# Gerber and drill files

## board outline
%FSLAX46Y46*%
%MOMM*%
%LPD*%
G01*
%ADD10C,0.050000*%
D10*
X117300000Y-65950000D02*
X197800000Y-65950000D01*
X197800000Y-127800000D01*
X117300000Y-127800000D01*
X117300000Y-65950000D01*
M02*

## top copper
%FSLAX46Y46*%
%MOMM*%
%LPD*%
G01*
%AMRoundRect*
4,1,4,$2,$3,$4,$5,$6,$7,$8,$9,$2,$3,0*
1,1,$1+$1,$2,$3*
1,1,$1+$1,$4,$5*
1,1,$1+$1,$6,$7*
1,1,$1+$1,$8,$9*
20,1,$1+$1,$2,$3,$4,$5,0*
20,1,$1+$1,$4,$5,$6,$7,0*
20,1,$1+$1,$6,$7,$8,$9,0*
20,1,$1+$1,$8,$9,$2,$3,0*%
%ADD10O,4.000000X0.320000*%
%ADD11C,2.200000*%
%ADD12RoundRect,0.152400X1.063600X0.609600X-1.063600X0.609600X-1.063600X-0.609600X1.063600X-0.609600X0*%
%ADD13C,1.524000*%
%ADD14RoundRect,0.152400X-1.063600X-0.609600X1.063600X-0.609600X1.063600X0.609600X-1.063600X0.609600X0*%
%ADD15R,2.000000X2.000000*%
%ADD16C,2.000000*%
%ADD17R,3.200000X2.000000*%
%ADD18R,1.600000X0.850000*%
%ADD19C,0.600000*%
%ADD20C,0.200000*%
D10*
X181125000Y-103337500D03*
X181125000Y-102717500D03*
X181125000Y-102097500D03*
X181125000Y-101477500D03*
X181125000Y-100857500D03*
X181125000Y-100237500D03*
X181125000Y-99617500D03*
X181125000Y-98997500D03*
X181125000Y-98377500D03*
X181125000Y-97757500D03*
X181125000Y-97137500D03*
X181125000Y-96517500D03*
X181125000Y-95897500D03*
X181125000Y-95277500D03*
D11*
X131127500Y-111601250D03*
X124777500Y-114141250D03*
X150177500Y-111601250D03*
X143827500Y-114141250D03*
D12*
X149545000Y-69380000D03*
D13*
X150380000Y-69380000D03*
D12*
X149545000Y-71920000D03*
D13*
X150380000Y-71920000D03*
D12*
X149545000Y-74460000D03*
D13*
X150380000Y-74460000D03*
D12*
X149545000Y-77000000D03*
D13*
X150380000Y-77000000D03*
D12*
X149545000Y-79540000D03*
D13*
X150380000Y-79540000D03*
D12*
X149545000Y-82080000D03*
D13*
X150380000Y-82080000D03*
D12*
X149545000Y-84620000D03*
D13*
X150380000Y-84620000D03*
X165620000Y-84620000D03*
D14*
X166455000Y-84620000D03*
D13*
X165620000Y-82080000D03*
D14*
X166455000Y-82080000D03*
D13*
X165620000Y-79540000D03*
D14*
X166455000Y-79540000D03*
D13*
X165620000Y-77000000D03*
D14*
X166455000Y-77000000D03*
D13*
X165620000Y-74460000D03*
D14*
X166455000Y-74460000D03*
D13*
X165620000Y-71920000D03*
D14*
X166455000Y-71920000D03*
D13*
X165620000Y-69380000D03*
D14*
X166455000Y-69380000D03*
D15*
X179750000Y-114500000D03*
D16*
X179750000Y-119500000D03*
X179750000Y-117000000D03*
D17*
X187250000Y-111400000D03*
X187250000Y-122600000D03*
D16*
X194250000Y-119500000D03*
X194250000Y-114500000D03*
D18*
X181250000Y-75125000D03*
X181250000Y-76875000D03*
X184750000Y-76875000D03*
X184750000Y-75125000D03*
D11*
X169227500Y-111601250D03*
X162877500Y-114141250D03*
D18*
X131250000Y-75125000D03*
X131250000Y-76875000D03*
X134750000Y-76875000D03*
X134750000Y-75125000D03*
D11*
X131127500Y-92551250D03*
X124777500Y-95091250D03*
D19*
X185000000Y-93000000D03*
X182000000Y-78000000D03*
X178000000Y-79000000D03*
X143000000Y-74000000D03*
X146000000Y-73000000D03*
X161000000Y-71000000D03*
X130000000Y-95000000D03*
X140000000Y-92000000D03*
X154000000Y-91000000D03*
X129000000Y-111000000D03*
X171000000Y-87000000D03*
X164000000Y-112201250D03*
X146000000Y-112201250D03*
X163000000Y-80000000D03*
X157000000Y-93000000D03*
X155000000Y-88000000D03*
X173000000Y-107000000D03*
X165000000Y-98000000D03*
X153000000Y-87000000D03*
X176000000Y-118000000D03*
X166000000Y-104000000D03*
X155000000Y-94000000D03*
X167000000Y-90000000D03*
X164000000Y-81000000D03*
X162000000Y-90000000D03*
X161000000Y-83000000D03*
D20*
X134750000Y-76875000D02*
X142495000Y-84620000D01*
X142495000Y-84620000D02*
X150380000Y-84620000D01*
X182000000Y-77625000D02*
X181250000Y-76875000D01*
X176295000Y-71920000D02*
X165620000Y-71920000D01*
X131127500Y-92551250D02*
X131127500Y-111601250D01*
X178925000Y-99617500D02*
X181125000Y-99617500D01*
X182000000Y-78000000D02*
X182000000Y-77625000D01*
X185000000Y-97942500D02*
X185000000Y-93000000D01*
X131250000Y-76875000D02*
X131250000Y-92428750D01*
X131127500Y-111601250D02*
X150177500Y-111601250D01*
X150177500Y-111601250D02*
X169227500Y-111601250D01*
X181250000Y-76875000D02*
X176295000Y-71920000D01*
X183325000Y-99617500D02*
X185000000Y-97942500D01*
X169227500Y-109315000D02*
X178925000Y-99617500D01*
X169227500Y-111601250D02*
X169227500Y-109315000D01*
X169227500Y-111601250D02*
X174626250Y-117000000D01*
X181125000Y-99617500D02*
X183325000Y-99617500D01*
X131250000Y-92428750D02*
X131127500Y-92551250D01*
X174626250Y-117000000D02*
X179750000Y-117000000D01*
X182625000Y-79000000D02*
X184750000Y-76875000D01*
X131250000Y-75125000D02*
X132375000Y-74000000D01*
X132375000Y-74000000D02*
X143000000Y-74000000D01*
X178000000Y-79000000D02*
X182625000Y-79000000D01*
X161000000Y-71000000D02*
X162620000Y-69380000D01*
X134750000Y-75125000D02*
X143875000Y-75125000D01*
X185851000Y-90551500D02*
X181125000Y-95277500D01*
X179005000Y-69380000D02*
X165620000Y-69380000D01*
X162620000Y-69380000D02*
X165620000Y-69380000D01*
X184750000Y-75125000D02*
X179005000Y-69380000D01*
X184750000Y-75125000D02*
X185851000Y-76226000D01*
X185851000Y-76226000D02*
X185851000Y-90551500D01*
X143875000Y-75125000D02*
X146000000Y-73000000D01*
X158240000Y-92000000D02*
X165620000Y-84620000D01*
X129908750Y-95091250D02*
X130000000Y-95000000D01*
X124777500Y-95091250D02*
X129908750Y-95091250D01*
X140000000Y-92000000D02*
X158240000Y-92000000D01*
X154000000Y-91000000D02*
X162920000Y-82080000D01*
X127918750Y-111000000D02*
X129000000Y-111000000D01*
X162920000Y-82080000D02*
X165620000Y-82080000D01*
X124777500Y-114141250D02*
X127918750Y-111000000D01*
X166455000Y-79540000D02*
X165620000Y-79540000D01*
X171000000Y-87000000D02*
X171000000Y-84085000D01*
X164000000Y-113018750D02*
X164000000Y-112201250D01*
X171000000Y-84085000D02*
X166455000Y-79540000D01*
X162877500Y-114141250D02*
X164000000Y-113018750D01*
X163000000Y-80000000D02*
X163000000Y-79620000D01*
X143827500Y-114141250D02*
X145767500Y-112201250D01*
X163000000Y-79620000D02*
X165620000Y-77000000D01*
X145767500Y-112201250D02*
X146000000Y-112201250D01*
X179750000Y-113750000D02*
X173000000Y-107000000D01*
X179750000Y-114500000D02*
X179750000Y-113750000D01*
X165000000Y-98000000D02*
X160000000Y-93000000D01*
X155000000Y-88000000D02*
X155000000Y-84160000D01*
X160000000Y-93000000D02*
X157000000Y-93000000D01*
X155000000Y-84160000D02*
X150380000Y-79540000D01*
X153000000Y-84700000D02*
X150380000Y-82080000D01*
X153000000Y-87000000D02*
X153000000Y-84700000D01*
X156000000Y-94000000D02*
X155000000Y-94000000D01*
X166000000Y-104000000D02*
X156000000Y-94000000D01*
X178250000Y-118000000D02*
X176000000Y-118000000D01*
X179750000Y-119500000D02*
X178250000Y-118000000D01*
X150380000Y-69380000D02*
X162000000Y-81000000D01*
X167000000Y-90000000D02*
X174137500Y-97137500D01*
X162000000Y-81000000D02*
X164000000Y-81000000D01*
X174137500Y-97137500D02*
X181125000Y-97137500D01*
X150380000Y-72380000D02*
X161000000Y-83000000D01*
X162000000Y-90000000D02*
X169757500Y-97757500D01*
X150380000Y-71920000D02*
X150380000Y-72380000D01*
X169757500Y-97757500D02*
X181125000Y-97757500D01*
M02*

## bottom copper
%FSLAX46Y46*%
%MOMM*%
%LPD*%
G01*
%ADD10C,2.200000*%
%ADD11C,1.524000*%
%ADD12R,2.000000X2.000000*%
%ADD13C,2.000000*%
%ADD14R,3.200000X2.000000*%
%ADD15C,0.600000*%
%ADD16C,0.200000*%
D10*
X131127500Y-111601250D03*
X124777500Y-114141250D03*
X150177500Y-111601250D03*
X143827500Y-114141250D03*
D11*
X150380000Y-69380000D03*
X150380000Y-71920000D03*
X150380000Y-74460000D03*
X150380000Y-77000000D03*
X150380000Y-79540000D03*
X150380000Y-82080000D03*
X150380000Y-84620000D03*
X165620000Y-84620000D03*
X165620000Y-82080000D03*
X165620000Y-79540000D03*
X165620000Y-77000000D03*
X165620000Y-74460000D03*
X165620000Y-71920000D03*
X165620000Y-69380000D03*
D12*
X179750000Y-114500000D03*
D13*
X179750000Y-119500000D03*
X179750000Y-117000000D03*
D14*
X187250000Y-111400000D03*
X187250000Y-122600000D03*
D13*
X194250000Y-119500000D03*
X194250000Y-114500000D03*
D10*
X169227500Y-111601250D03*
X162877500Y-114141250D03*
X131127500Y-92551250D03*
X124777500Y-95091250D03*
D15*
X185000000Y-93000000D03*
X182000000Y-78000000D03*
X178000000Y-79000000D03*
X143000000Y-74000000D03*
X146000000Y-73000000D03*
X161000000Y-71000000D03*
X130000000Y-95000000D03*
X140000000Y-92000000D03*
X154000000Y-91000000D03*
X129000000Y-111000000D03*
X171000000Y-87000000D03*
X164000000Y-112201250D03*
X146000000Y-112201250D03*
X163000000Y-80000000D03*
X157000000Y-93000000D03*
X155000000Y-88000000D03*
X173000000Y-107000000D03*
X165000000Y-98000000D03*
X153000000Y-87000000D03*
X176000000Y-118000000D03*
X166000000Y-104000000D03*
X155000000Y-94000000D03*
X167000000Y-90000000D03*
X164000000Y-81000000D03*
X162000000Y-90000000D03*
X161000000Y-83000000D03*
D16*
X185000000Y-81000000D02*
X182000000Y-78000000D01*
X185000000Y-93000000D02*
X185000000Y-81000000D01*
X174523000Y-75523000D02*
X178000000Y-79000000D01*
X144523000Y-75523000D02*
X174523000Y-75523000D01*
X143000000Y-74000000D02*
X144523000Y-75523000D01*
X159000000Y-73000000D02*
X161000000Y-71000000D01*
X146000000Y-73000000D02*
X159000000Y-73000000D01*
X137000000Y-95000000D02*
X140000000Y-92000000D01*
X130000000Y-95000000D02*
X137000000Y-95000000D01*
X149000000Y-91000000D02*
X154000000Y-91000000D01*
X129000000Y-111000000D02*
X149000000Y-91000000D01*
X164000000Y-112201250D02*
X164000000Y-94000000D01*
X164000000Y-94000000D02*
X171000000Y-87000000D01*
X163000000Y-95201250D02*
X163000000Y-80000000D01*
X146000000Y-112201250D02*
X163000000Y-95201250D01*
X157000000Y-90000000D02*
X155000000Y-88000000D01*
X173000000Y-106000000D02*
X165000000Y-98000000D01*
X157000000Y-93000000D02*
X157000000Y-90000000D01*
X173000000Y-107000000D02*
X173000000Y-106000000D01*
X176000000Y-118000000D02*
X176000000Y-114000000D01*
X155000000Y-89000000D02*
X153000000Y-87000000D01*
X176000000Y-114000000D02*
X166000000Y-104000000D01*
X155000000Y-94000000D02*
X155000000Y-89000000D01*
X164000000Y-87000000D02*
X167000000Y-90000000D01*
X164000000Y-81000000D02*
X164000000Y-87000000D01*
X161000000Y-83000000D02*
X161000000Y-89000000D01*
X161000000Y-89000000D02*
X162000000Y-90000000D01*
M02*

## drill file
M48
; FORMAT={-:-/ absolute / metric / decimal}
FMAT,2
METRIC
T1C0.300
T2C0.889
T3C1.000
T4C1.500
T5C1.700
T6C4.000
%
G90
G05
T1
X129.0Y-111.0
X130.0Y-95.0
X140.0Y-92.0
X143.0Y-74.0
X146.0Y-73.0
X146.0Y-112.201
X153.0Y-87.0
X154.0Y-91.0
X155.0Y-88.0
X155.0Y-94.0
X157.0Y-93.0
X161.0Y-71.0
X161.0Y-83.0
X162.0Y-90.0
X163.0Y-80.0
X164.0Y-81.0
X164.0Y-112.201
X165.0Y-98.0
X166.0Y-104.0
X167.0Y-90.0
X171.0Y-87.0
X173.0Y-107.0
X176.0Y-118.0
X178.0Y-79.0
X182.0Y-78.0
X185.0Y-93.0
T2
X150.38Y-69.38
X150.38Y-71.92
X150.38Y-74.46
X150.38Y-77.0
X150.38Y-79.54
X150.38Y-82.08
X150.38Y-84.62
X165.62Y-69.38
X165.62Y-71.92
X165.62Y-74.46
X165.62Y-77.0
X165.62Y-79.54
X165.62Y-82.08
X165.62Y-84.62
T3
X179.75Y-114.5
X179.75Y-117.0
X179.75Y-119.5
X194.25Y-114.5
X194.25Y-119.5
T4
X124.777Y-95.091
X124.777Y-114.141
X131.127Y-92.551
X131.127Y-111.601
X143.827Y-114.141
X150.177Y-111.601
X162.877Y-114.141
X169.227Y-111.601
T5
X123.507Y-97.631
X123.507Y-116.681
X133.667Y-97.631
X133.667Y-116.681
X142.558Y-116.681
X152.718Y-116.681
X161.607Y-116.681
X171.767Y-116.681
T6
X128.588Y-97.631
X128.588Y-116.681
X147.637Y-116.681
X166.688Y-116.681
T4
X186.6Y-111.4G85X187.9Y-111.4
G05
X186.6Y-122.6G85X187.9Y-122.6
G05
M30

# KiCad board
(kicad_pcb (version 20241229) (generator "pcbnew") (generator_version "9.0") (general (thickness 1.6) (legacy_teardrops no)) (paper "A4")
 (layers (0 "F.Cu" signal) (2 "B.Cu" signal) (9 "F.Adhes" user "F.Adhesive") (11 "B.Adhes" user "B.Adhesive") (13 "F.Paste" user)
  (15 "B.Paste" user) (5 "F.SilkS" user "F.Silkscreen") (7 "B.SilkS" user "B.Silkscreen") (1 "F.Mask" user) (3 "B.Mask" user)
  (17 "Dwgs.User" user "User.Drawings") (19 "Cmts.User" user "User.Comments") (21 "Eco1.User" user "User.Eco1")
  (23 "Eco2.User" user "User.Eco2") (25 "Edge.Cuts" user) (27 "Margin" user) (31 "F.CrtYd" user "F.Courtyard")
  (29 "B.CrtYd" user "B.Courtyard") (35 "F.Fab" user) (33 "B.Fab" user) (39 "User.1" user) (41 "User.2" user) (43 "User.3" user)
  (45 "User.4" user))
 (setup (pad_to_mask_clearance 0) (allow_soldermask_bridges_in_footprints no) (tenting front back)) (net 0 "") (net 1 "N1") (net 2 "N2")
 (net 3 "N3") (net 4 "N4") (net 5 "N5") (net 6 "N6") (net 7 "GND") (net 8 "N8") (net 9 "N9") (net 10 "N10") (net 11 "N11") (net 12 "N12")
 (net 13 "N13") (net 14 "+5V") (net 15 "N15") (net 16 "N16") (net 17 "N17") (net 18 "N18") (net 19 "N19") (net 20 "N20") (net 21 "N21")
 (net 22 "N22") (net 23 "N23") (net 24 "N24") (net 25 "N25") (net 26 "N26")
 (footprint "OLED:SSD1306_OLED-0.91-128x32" (layer "F.Cu") (at 141.125 92.3375)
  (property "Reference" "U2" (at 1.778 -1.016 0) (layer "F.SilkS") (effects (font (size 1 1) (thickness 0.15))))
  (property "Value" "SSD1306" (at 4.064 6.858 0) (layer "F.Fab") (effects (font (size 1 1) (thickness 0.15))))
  (pad "1" smd oval (at 40 11) (size 4 0.32) (layers "F.Cu" "F.Mask" "F.Paste") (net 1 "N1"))
  (pad "2" smd oval (at 40 10.38) (size 4 0.32) (layers "F.Cu" "F.Mask" "F.Paste") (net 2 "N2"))
  (pad "3" smd oval (at 40 9.76) (size 4 0.32) (layers "F.Cu" "F.Mask" "F.Paste") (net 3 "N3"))
  (pad "4" smd oval (at 40 9.14) (size 4 0.32) (layers "F.Cu" "F.Mask" "F.Paste") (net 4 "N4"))
  (pad "5" smd oval (at 40 8.52) (size 4 0.32) (layers "F.Cu" "F.Mask" "F.Paste") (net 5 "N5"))
  (pad "6" smd oval (at 40 7.9) (size 4 0.32) (layers "F.Cu" "F.Mask" "F.Paste") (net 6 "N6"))
  (pad "7" smd oval (at 40 7.28) (size 4 0.32) (layers "F.Cu" "F.Mask" "F.Paste") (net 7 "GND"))
  (pad "8" smd oval (at 40 6.66) (size 4 0.32) (layers "F.Cu" "F.Mask" "F.Paste") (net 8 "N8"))
  (pad "9" smd oval (at 40 6.04) (size 4 0.32) (layers "F.Cu" "F.Mask" "F.Paste") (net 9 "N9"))
  (pad "10" smd oval (at 40 5.42) (size 4 0.32) (layers "F.Cu" "F.Mask" "F.Paste") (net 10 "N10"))
  (pad "11" smd oval (at 40 4.8) (size 4 0.32) (layers "F.Cu" "F.Mask" "F.Paste") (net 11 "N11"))
  (pad "12" smd oval (at 40 4.18) (size 4 0.32) (layers "F.Cu" "F.Mask" "F.Paste") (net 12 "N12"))
  (pad "13" smd oval (at 40 3.56) (size 4 0.32) (layers "F.Cu" "F.Mask" "F.Paste") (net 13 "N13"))
  (pad "14" smd oval (at 40 2.94) (size 4 0.32) (layers "F.Cu" "F.Mask" "F.Paste") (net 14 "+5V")))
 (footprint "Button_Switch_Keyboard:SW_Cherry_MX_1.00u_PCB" (layer "F.Cu") (at 131.1275 111.60125)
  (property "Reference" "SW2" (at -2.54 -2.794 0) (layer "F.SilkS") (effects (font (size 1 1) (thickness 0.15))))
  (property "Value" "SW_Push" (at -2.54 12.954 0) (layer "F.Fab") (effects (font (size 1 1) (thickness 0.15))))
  (pad "" np_thru_hole circle (at -7.62 5.08) (size 1.7 1.7) (drill 1.7) (layers "*.Cu" "*.Mask"))
  (pad "" np_thru_hole circle (at -2.54 5.08) (size 4 4) (drill 4) (layers "*.Cu" "*.Mask"))
  (pad "" np_thru_hole circle (at 2.54 5.08) (size 1.7 1.7) (drill 1.7) (layers "*.Cu" "*.Mask"))
  (pad "1" thru_hole circle (at 0 0) (size 2.2 2.2) (drill 1.5) (layers "*.Cu" "*.Mask") (remove_unused_layers no) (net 7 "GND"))
  (pad "2" thru_hole circle (at -6.35 2.54) (size 2.2 2.2) (drill 1.5) (layers "*.Cu" "*.Mask") (remove_unused_layers no) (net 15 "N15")))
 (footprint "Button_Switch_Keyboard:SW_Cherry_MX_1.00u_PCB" (layer "F.Cu") (at 150.1775 111.60125)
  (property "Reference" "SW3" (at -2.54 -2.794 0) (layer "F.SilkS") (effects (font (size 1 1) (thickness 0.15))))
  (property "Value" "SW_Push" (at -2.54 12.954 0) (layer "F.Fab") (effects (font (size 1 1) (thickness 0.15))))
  (pad "" np_thru_hole circle (at -7.62 5.08) (size 1.7 1.7) (drill 1.7) (layers "*.Cu" "*.Mask"))
  (pad "" np_thru_hole circle (at -2.54 5.08) (size 4 4) (drill 4) (layers "*.Cu" "*.Mask"))
  (pad "" np_thru_hole circle (at 2.54 5.08) (size 1.7 1.7) (drill 1.7) (layers "*.Cu" "*.Mask"))
  (pad "1" thru_hole circle (at 0 0) (size 2.2 2.2) (drill 1.5) (layers "*.Cu" "*.Mask") (remove_unused_layers no) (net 7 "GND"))
  (pad "2" thru_hole circle (at -6.35 2.54) (size 2.2 2.2) (drill 1.5) (layers "*.Cu" "*.Mask") (remove_unused_layers no) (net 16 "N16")))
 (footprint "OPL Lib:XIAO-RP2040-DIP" (layer "F.Cu") (at 158 77)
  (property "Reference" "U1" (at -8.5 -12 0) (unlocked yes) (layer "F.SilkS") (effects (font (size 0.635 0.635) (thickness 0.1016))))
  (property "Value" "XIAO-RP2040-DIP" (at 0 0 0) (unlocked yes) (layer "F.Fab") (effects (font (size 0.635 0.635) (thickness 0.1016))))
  (pad "1" smd roundrect (at -8.455 -7.62 180) (size 2.432 1.524) (layers "F.Cu" "F.Mask") (roundrect_rratio 0.1) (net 11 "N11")
   (thermal_bridge_angle 45))
  (pad "1" thru_hole circle (at -7.62 -7.62 180) (size 1.524 1.524) (drill 0.889) (layers "*.Cu" "*.Mask") (remove_unused_layers no)
   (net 11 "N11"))
  (pad "2" smd roundrect (at -8.455 -5.08 180) (size 2.432 1.524) (layers "F.Cu" "F.Mask") (roundrect_rratio 0.1) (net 10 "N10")
   (thermal_bridge_angle 45))
  (pad "2" thru_hole circle (at -7.62 -5.08 180) (size 1.524 1.524) (drill 0.889) (layers "*.Cu" "*.Mask") (remove_unused_layers no)
   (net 10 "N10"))
  (pad "3" smd roundrect (at -8.455 -2.54 180) (size 2.432 1.524) (layers "F.Cu" "F.Mask") (roundrect_rratio 0.1) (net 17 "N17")
   (thermal_bridge_angle 45))
  (pad "3" thru_hole circle (at -7.62 -2.54 180) (size 1.524 1.524) (drill 0.889) (layers "*.Cu" "*.Mask") (remove_unused_layers no)
   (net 17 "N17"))
  (pad "4" smd roundrect (at -8.455 0 180) (size 2.432 1.524) (layers "F.Cu" "F.Mask") (roundrect_rratio 0.1) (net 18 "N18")
   (thermal_bridge_angle 45))
  (pad "4" thru_hole circle (at -7.62 0 180) (size 1.524 1.524) (drill 0.889) (layers "*.Cu" "*.Mask") (remove_unused_layers no)
   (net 18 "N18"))
  (pad "5" smd roundrect (at -8.455 2.54 180) (size 2.432 1.524) (layers "F.Cu" "F.Mask") (roundrect_rratio 0.1) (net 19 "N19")
   (thermal_bridge_angle 45))
  (pad "5" thru_hole circle (at -7.62 2.54 180) (size 1.524 1.524) (drill 0.889) (layers "*.Cu" "*.Mask") (remove_unused_layers no)
   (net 19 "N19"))
  (pad "6" smd roundrect (at -8.455 5.08 180) (size 2.432 1.524) (layers "F.Cu" "F.Mask") (roundrect_rratio 0.1) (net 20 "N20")
   (thermal_bridge_angle 45))
  (pad "6" thru_hole circle (at -7.62 5.08 180) (size 1.524 1.524) (drill 0.889) (layers "*.Cu" "*.Mask") (remove_unused_layers no)
   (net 20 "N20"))
  (pad "7" smd roundrect (at -8.455 7.62 180) (size 2.432 1.524) (layers "F.Cu" "F.Mask") (roundrect_rratio 0.1) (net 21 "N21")
   (thermal_bridge_angle 45))
  (pad "7" thru_hole circle (at -7.62 7.62 180) (size 1.524 1.524) (drill 0.889) (layers "*.Cu" "*.Mask") (remove_unused_layers no)
   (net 21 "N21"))
  (pad "8" thru_hole circle (at 7.62 7.62) (size 1.524 1.524) (drill 0.889) (layers "*.Cu" "*.Mask") (remove_unused_layers no)
   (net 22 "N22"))
  (pad "8" smd roundrect (at 8.455 7.62) (size 2.432 1.524) (layers "F.Cu" "F.Mask") (roundrect_rratio 0.1) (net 22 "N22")
   (thermal_bridge_angle 45))
  (pad "9" thru_hole circle (at 7.62 5.08) (size 1.524 1.524) (drill 0.889) (layers "*.Cu" "*.Mask") (remove_unused_layers no)
   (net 15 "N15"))
  (pad "9" smd roundrect (at 8.455 5.08) (size 2.432 1.524) (layers "F.Cu" "F.Mask") (roundrect_rratio 0.1) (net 15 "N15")
   (thermal_bridge_angle 45))
  (pad "10" thru_hole circle (at 7.62 2.54) (size 1.524 1.524) (drill 0.889) (layers "*.Cu" "*.Mask") (remove_unused_layers no)
   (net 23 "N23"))
  (pad "10" smd roundrect (at 8.455 2.54) (size 2.432 1.524) (layers "F.Cu" "F.Mask") (roundrect_rratio 0.1) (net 23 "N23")
   (thermal_bridge_angle 45))
  (pad "11" thru_hole circle (at 7.62 0) (size 1.524 1.524) (drill 0.889) (layers "*.Cu" "*.Mask") (remove_unused_layers no) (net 16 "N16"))
  (pad "11" smd roundrect (at 8.455 0) (size 2.432 1.524) (layers "F.Cu" "F.Mask") (roundrect_rratio 0.1) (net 16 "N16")
   (thermal_bridge_angle 45))
  (pad "12" thru_hole circle (at 7.62 -2.54) (size 1.524 1.524) (drill 0.889) (layers "*.Cu" "*.Mask") (remove_unused_layers no)
   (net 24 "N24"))
  (pad "12" smd roundrect (at 8.455 -2.54) (size 2.432 1.524) (layers "F.Cu" "F.Mask") (roundrect_rratio 0.1) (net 24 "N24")
   (thermal_bridge_angle 45))
  (pad "13" thru_hole circle (at 7.62 -5.08) (size 1.524 1.524) (drill 0.889) (layers "*.Cu" "*.Mask") (remove_unused_layers no)
   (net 7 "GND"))
  (pad "13" smd roundrect (at 8.455 -5.08) (size 2.432 1.524) (layers "F.Cu" "F.Mask") (roundrect_rratio 0.1) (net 7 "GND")
   (thermal_bridge_angle 45))
  (pad "14" thru_hole circle (at 7.62 -7.62) (size 1.524 1.524) (drill 0.889) (layers "*.Cu" "*.Mask") (remove_unused_layers no)
   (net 14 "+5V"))
  (pad "14" smd roundrect (at 8.455 -7.62) (size 2.432 1.524) (layers "F.Cu" "F.Mask") (roundrect_rratio 0.1) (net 14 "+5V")
   (thermal_bridge_angle 45)))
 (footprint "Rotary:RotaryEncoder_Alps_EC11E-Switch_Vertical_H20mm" (layer "F.Cu") (at 179.75 114.5)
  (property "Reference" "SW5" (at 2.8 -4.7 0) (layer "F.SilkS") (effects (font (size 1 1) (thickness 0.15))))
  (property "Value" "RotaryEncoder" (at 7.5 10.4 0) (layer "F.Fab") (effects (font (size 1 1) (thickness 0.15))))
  (pad "A" thru_hole rect (at 0 0) (size 2 2) (drill 1) (layers "*.Cu" "*.Mask") (remove_unused_layers no) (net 19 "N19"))
  (pad "B" thru_hole circle (at 0 5) (size 2 2) (drill 1) (layers "*.Cu" "*.Mask") (remove_unused_layers no) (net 20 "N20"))
  (pad "C" thru_hole circle (at 0 2.5) (size 2 2) (drill 1) (layers "*.Cu" "*.Mask") (remove_unused_layers no) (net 7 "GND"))
  (pad "MP" thru_hole rect (at 7.5 -3.1) (size 3.2 2) (drill oval 2.8 1.5) (layers "*.Cu" "*.Mask") (remove_unused_layers no))
  (pad "MP" thru_hole rect (at 7.5 8.1) (size 3.2 2) (drill oval 2.8 1.5) (layers "*.Cu" "*.Mask") (remove_unused_layers no))
  (pad "S1" thru_hole circle (at 14.5 5) (size 2 2) (drill 1) (layers "*.Cu" "*.Mask") (remove_unused_layers no))
  (pad "S2" thru_hole circle (at 14.5 0) (size 2 2) (drill 1) (layers "*.Cu" "*.Mask") (remove_unused_layers no)))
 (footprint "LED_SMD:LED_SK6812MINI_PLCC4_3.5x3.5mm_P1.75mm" (layer "F.Cu") (at 183 76)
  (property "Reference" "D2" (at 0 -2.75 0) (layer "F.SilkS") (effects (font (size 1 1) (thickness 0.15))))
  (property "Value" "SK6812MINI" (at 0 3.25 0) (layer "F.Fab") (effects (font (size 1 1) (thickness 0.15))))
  (pad "1" smd rect (at -1.75 -0.875) (size 1.6 0.85) (layers "F.Cu" "F.Mask" "F.Paste") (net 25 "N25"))
  (pad "2" smd rect (at -1.75 0.875) (size 1.6 0.85) (layers "F.Cu" "F.Mask" "F.Paste") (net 7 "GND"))
  (pad "3" smd rect (at 1.75 0.875) (size 1.6 0.85) (layers "F.Cu" "F.Mask" "F.Paste") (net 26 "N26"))
  (pad "4" smd rect (at 1.75 -0.875) (size 1.6 0.85) (layers "F.Cu" "F.Mask" "F.Paste") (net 14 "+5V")))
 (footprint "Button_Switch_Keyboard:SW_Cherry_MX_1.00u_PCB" (layer "F.Cu") (at 169.2275 111.60125)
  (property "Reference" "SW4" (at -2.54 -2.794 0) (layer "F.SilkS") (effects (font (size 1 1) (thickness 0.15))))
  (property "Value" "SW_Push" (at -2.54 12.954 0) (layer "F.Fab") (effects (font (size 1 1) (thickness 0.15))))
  (pad "" np_thru_hole circle (at -7.62 5.08) (size 1.7 1.7) (drill 1.7) (layers "*.Cu" "*.Mask"))
  (pad "" np_thru_hole circle (at -2.54 5.08) (size 4 4) (drill 4) (layers "*.Cu" "*.Mask"))
  (pad "" np_thru_hole circle (at 2.54 5.08) (size 1.7 1.7) (drill 1.7) (layers "*.Cu" "*.Mask"))
  (pad "1" thru_hole circle (at 0 0) (size 2.2 2.2) (drill 1.5) (layers "*.Cu" "*.Mask") (remove_unused_layers no) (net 7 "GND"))
  (pad "2" thru_hole circle (at -6.35 2.54) (size 2.2 2.2) (drill 1.5) (layers "*.Cu" "*.Mask") (remove_unused_layers no) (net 23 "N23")))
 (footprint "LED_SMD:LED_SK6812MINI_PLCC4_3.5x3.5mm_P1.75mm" (layer "F.Cu") (at 133 76)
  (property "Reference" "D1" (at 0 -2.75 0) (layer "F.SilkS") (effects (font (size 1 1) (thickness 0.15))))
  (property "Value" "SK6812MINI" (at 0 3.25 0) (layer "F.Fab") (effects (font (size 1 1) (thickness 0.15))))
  (pad "1" smd rect (at -1.75 -0.875) (size 1.6 0.85) (layers "F.Cu" "F.Mask" "F.Paste") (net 26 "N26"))
  (pad "2" smd rect (at -1.75 0.875) (size 1.6 0.85) (layers "F.Cu" "F.Mask" "F.Paste") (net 7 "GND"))
  (pad "3" smd rect (at 1.75 0.875) (size 1.6 0.85) (layers "F.Cu" "F.Mask" "F.Paste") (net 21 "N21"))
  (pad "4" smd rect (at 1.75 -0.875) (size 1.6 0.85) (layers "F.Cu" "F.Mask" "F.Paste") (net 14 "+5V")))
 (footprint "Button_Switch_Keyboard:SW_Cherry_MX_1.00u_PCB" (layer "F.Cu") (at 131.1275 92.55125)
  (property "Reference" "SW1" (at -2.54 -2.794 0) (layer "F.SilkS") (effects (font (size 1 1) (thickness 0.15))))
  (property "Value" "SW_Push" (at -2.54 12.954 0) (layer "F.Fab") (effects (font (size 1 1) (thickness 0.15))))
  (pad "" np_thru_hole circle (at -7.62 5.08) (size 1.7 1.7) (drill 1.7) (layers "*.Cu" "*.Mask"))
  (pad "" np_thru_hole circle (at -2.54 5.08) (size 4 4) (drill 4) (layers "*.Cu" "*.Mask"))
  (pad "" np_thru_hole circle (at 2.54 5.08) (size 1.7 1.7) (drill 1.7) (layers "*.Cu" "*.Mask"))
  (pad "1" thru_hole circle (at 0 0) (size 2.2 2.2) (drill 1.5) (layers "*.Cu" "*.Mask") (remove_unused_layers no) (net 7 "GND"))
  (pad "2" thru_hole circle (at -6.35 2.54) (size 2.2 2.2) (drill 1.5) (layers "*.Cu" "*.Mask") (remove_unused_layers no) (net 22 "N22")))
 (gr_rect (start 117.3 65.95) (end 197.8 127.8) (stroke (width 0.05) (type default)) (fill no) (layer "Edge.Cuts"))
 (segment (start 134.75 76.875) (end 142.495 84.62) (width 0.2) (layer "F.Cu") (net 21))
 (segment (start 142.495 84.62) (end 150.38 84.62) (width 0.2) (layer "F.Cu") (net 21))
 (segment (start 182 77.625) (end 181.25 76.875) (width 0.2) (layer "F.Cu") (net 7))
 (segment (start 176.295 71.92) (end 165.62 71.92) (width 0.2) (layer "F.Cu") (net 7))
 (segment (start 131.1275 92.55125) (end 131.1275 111.60125) (width 0.2) (layer "F.Cu") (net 7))
 (segment (start 178.925 99.6175) (end 181.125 99.6175) (width 0.2) (layer "F.Cu") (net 7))
 (segment (start 182 78) (end 182 77.625) (width 0.2) (layer "F.Cu") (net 7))
 (segment (start 185 97.9425) (end 185 93) (width 0.2) (layer "F.Cu") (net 7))
 (segment (start 131.25 76.875) (end 131.25 92.42875) (width 0.2) (layer "F.Cu") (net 7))
 (segment (start 131.1275 111.60125) (end 150.1775 111.60125) (width 0.2) (layer "F.Cu") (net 7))
 (segment (start 150.1775 111.60125) (end 169.2275 111.60125) (width 0.2) (layer "F.Cu") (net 7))
 (segment (start 181.25 76.875) (end 176.295 71.92) (width 0.2) (layer "F.Cu") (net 7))
 (segment (start 183.325 99.6175) (end 185 97.9425) (width 0.2) (layer "F.Cu") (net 7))
 (segment (start 169.2275 109.315) (end 178.925 99.6175) (width 0.2) (layer "F.Cu") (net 7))
 (segment (start 169.2275 111.60125) (end 169.2275 109.315) (width 0.2) (layer "F.Cu") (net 7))
 (segment (start 169.2275 111.60125) (end 174.62625 117) (width 0.2) (layer "F.Cu") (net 7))
 (segment (start 181.125 99.6175) (end 183.325 99.6175) (width 0.2) (layer "F.Cu") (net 7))
 (segment (start 131.25 92.42875) (end 131.1275 92.55125) (width 0.2) (layer "F.Cu") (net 7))
 (segment (start 174.62625 117) (end 179.75 117) (width 0.2) (layer "F.Cu") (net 7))
 (via (at 185 93) (size 0.6) (drill 0.3) (layers "F.Cu" "B.Cu") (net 7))
 (via (at 182 78) (size 0.6) (drill 0.3) (layers "F.Cu" "B.Cu") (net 7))
 (segment (start 185 81) (end 182 78) (width 0.2) (layer "B.Cu") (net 7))
 (segment (start 185 93) (end 185 81) (width 0.2) (layer "B.Cu") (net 7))
 (segment (start 182.625 79) (end 184.75 76.875) (width 0.2) (layer "F.Cu") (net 26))
 (segment (start 131.25 75.125) (end 132.375 74) (width 0.2) (layer "F.Cu") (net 26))
 (segment (start 132.375 74) (end 143 74) (width 0.2) (layer "F.Cu") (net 26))
 (segment (start 178 79) (end 182.625 79) (width 0.2) (layer "F.Cu") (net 26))
 (via (at 178 79) (size 0.6) (drill 0.3) (layers "F.Cu" "B.Cu") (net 26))
 (via (at 143 74) (size 0.6) (drill 0.3) (layers "F.Cu" "B.Cu") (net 26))
 (segment (start 174.523 75.523) (end 178 79) (width 0.2) (layer "B.Cu") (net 26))
 (segment (start 144.523 75.523) (end 174.523 75.523) (width 0.2) (layer "B.Cu") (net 26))
 (segment (start 143 74) (end 144.523 75.523) (width 0.2) (layer "B.Cu") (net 26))
 (segment (start 161 71) (end 162.62 69.38) (width 0.2) (layer "F.Cu") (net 14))
 (segment (start 134.75 75.125) (end 143.875 75.125) (width 0.2) (layer "F.Cu") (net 14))
 (segment (start 185.851 90.5515) (end 181.125 95.2775) (width 0.2) (layer "F.Cu") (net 14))
 (segment (start 179.005 69.38) (end 165.62 69.38) (width 0.2) (layer "F.Cu") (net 14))
 (segment (start 162.62 69.38) (end 165.62 69.38) (width 0.2) (layer "F.Cu") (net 14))
 (segment (start 184.75 75.125) (end 179.005 69.38) (width 0.2) (layer "F.Cu") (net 14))
 (segment (start 184.75 75.125) (end 185.851 76.226) (width 0.2) (layer "F.Cu") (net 14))
 (segment (start 185.851 76.226) (end 185.851 90.5515) (width 0.2) (layer "F.Cu") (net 14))
 (segment (start 143.875 75.125) (end 146 73) (width 0.2) (layer "F.Cu") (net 14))
 (via (at 146 73) (size 0.6) (drill 0.3) (layers "F.Cu" "B.Cu") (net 14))
 (via (at 161 71) (size 0.6) (drill 0.3) (layers "F.Cu" "B.Cu") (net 14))
 (segment (start 159 73) (end 161 71) (width 0.2) (layer "B.Cu") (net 14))
 (segment (start 146 73) (end 159 73) (width 0.2) (layer "B.Cu") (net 14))
 (segment (start 158.24 92) (end 165.62 84.62) (width 0.2) (layer "F.Cu") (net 22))
 (segment (start 129.90875 95.09125) (end 130 95) (width 0.2) (layer "F.Cu") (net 22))
 (segment (start 124.7775 95.09125) (end 129.90875 95.09125) (width 0.2) (layer "F.Cu") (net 22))
 (segment (start 140 92) (end 158.24 92) (width 0.2) (layer "F.Cu") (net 22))
 (via (at 130 95) (size 0.6) (drill 0.3) (layers "F.Cu" "B.Cu") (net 22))
 (via (at 140 92) (size 0.6) (drill 0.3) (layers "F.Cu" "B.Cu") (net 22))
 (segment (start 137 95) (end 140 92) (width 0.2) (layer "B.Cu") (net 22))
 (segment (start 130 95) (end 137 95) (width 0.2) (layer "B.Cu") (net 22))
 (segment (start 154 91) (end 162.92 82.08) (width 0.2) (layer "F.Cu") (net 15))
 (segment (start 127.91875 111) (end 129 111) (width 0.2) (layer "F.Cu") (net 15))
 (segment (start 162.92 82.08) (end 165.62 82.08) (width 0.2) (layer "F.Cu") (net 15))
 (segment (start 124.7775 114.14125) (end 127.91875 111) (width 0.2) (layer "F.Cu") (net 15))
 (via (at 154 91) (size 0.6) (drill 0.3) (layers "F.Cu" "B.Cu") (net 15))
 (via (at 129 111) (size 0.6) (drill 0.3) (layers "F.Cu" "B.Cu") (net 15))
 (segment (start 149 91) (end 154 91) (width 0.2) (layer "B.Cu") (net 15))
 (segment (start 129 111) (end 149 91) (width 0.2) (layer "B.Cu") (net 15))
 (segment (start 166.455 79.54) (end 165.62 79.54) (width 0.2) (layer "F.Cu") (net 23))
 (segment (start 171 87) (end 171 84.085) (width 0.2) (layer "F.Cu") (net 23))
 (segment (start 164 113.01875) (end 164 112.20125) (width 0.2) (layer "F.Cu") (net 23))
 (segment (start 171 84.085) (end 166.455 79.54) (width 0.2) (layer "F.Cu") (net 23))
 (segment (start 162.8775 114.14125) (end 164 113.01875) (width 0.2) (layer "F.Cu") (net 23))
 (via (at 171 87) (size 0.6) (drill 0.3) (layers "F.Cu" "B.Cu") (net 23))
 (via (at 164 112.20125) (size 0.6) (drill 0.3) (layers "F.Cu" "B.Cu") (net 23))
 (segment (start 164 112.20125) (end 164 94) (width 0.2) (layer "B.Cu") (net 23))
 (segment (start 164 94) (end 171 87) (width 0.2) (layer "B.Cu") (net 23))
 (segment (start 163 80) (end 163 79.62) (width 0.2) (layer "F.Cu") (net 16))
 (segment (start 143.8275 114.14125) (end 145.7675 112.20125) (width 0.2) (layer "F.Cu") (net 16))
 (segment (start 163 79.62) (end 165.62 77) (width 0.2) (layer "F.Cu") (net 16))
 (segment (start 145.7675 112.20125) (end 146 112.20125) (width 0.2) (layer "F.Cu") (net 16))
 (via (at 146 112.20125) (size 0.6) (drill 0.3) (layers "F.Cu" "B.Cu") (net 16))
 (via (at 163 80) (size 0.6) (drill 0.3) (layers "F.Cu" "B.Cu") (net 16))
 (segment (start 163 95.20125) (end 163 80) (width 0.2) (layer "B.Cu") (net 16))
 (segment (start 146 112.20125) (end 163 95.20125) (width 0.2) (layer "B.Cu") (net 16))
 (segment (start 179.75 113.75) (end 173 107) (width 0.2) (layer "F.Cu") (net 19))
 (segment (start 179.75 114.5) (end 179.75 113.75) (width 0.2) (layer "F.Cu") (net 19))
 (segment (start 165 98) (end 160 93) (width 0.2) (layer "F.Cu") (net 19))
 (segment (start 155 88) (end 155 84.16) (width 0.2) (layer "F.Cu") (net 19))
 (segment (start 160 93) (end 157 93) (width 0.2) (layer "F.Cu") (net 19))
 (segment (start 155 84.16) (end 150.38 79.54) (width 0.2) (layer "F.Cu") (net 19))
 (via (at 157 93) (size 0.6) (drill 0.3) (layers "F.Cu" "B.Cu") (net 19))
 (via (at 155 88) (size 0.6) (drill 0.3) (layers "F.Cu" "B.Cu") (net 19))
 (via (at 173 107) (size 0.6) (drill 0.3) (layers "F.Cu" "B.Cu") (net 19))
 (via (at 165 98) (size 0.6) (drill 0.3) (layers "F.Cu" "B.Cu") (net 19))
 (segment (start 157 90) (end 155 88) (width 0.2) (layer "B.Cu") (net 19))
 (segment (start 173 106) (end 165 98) (width 0.2) (layer "B.Cu") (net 19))
 (segment (start 157 93) (end 157 90) (width 0.2) (layer "B.Cu") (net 19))
 (segment (start 173 107) (end 173 106) (width 0.2) (layer "B.Cu") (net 19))
 (segment (start 153 84.7) (end 150.38 82.08) (width 0.2) (layer "F.Cu") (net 20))
 (segment (start 153 87) (end 153 84.7) (width 0.2) (layer "F.Cu") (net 20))
 (segment (start 156 94) (end 155 94) (width 0.2) (layer "F.Cu") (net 20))
 (segment (start 166 104) (end 156 94) (width 0.2) (layer "F.Cu") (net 20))
 (segment (start 178.25 118) (end 176 118) (width 0.2) (layer "F.Cu") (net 20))
 (segment (start 179.75 119.5) (end 178.25 118) (width 0.2) (layer "F.Cu") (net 20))
 (via (at 153 87) (size 0.6) (drill 0.3) (layers "F.Cu" "B.Cu") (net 20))
 (via (at 176 118) (size 0.6) (drill 0.3) (layers "F.Cu" "B.Cu") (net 20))
 (via (at 166 104) (size 0.6) (drill 0.3) (layers "F.Cu" "B.Cu") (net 20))
 (via (at 155 94) (size 0.6) (drill 0.3) (layers "F.Cu" "B.Cu") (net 20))
 (segment (start 176 118) (end 176 114) (width 0.2) (layer "B.Cu") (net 20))
 (segment (start 155 89) (end 153 87) (width 0.2) (layer "B.Cu") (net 20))
 (segment (start 176 114) (end 166 104) (width 0.2) (layer "B.Cu") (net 20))
 (segment (start 155 94) (end 155 89) (width 0.2) (layer "B.Cu") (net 20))
 (segment (start 150.38 69.38) (end 162 81) (width 0.2) (layer "F.Cu") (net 11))
 (segment (start 167 90) (end 174.1375 97.1375) (width 0.2) (layer "F.Cu") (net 11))
 (segment (start 162 81) (end 164 81) (width 0.2) (layer "F.Cu") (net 11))
 (segment (start 174.1375 97.1375) (end 181.125 97.1375) (width 0.2) (layer "F.Cu") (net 11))
 (via (at 167 90) (size 0.6) (drill 0.3) (layers "F.Cu" "B.Cu") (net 11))
 (via (at 164 81) (size 0.6) (drill 0.3) (layers "F.Cu" "B.Cu") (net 11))
 (segment (start 164 87) (end 167 90) (width 0.2) (layer "B.Cu") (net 11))
 (segment (start 164 81) (end 164 87) (width 0.2) (layer "B.Cu") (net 11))
 (segment (start 150.38 72.38) (end 161 83) (width 0.2) (layer "F.Cu") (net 10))
 (segment (start 162 90) (end 169.7575 97.7575) (width 0.2) (layer "F.Cu") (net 10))
 (segment (start 150.38 71.92) (end 150.38 72.38) (width 0.2) (layer "F.Cu") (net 10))
 (segment (start 169.7575 97.7575) (end 181.125 97.7575) (width 0.2) (layer "F.Cu") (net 10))
 (via (at 162 90) (size 0.6) (drill 0.3) (layers "F.Cu" "B.Cu") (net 10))
 (via (at 161 83) (size 0.6) (drill 0.3) (layers "F.Cu" "B.Cu") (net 10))
 (segment (start 161 83) (end 161 89) (width 0.2) (layer "B.Cu") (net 10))
 (segment (start 161 89) (end 162 90) (width 0.2) (layer "B.Cu") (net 10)))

